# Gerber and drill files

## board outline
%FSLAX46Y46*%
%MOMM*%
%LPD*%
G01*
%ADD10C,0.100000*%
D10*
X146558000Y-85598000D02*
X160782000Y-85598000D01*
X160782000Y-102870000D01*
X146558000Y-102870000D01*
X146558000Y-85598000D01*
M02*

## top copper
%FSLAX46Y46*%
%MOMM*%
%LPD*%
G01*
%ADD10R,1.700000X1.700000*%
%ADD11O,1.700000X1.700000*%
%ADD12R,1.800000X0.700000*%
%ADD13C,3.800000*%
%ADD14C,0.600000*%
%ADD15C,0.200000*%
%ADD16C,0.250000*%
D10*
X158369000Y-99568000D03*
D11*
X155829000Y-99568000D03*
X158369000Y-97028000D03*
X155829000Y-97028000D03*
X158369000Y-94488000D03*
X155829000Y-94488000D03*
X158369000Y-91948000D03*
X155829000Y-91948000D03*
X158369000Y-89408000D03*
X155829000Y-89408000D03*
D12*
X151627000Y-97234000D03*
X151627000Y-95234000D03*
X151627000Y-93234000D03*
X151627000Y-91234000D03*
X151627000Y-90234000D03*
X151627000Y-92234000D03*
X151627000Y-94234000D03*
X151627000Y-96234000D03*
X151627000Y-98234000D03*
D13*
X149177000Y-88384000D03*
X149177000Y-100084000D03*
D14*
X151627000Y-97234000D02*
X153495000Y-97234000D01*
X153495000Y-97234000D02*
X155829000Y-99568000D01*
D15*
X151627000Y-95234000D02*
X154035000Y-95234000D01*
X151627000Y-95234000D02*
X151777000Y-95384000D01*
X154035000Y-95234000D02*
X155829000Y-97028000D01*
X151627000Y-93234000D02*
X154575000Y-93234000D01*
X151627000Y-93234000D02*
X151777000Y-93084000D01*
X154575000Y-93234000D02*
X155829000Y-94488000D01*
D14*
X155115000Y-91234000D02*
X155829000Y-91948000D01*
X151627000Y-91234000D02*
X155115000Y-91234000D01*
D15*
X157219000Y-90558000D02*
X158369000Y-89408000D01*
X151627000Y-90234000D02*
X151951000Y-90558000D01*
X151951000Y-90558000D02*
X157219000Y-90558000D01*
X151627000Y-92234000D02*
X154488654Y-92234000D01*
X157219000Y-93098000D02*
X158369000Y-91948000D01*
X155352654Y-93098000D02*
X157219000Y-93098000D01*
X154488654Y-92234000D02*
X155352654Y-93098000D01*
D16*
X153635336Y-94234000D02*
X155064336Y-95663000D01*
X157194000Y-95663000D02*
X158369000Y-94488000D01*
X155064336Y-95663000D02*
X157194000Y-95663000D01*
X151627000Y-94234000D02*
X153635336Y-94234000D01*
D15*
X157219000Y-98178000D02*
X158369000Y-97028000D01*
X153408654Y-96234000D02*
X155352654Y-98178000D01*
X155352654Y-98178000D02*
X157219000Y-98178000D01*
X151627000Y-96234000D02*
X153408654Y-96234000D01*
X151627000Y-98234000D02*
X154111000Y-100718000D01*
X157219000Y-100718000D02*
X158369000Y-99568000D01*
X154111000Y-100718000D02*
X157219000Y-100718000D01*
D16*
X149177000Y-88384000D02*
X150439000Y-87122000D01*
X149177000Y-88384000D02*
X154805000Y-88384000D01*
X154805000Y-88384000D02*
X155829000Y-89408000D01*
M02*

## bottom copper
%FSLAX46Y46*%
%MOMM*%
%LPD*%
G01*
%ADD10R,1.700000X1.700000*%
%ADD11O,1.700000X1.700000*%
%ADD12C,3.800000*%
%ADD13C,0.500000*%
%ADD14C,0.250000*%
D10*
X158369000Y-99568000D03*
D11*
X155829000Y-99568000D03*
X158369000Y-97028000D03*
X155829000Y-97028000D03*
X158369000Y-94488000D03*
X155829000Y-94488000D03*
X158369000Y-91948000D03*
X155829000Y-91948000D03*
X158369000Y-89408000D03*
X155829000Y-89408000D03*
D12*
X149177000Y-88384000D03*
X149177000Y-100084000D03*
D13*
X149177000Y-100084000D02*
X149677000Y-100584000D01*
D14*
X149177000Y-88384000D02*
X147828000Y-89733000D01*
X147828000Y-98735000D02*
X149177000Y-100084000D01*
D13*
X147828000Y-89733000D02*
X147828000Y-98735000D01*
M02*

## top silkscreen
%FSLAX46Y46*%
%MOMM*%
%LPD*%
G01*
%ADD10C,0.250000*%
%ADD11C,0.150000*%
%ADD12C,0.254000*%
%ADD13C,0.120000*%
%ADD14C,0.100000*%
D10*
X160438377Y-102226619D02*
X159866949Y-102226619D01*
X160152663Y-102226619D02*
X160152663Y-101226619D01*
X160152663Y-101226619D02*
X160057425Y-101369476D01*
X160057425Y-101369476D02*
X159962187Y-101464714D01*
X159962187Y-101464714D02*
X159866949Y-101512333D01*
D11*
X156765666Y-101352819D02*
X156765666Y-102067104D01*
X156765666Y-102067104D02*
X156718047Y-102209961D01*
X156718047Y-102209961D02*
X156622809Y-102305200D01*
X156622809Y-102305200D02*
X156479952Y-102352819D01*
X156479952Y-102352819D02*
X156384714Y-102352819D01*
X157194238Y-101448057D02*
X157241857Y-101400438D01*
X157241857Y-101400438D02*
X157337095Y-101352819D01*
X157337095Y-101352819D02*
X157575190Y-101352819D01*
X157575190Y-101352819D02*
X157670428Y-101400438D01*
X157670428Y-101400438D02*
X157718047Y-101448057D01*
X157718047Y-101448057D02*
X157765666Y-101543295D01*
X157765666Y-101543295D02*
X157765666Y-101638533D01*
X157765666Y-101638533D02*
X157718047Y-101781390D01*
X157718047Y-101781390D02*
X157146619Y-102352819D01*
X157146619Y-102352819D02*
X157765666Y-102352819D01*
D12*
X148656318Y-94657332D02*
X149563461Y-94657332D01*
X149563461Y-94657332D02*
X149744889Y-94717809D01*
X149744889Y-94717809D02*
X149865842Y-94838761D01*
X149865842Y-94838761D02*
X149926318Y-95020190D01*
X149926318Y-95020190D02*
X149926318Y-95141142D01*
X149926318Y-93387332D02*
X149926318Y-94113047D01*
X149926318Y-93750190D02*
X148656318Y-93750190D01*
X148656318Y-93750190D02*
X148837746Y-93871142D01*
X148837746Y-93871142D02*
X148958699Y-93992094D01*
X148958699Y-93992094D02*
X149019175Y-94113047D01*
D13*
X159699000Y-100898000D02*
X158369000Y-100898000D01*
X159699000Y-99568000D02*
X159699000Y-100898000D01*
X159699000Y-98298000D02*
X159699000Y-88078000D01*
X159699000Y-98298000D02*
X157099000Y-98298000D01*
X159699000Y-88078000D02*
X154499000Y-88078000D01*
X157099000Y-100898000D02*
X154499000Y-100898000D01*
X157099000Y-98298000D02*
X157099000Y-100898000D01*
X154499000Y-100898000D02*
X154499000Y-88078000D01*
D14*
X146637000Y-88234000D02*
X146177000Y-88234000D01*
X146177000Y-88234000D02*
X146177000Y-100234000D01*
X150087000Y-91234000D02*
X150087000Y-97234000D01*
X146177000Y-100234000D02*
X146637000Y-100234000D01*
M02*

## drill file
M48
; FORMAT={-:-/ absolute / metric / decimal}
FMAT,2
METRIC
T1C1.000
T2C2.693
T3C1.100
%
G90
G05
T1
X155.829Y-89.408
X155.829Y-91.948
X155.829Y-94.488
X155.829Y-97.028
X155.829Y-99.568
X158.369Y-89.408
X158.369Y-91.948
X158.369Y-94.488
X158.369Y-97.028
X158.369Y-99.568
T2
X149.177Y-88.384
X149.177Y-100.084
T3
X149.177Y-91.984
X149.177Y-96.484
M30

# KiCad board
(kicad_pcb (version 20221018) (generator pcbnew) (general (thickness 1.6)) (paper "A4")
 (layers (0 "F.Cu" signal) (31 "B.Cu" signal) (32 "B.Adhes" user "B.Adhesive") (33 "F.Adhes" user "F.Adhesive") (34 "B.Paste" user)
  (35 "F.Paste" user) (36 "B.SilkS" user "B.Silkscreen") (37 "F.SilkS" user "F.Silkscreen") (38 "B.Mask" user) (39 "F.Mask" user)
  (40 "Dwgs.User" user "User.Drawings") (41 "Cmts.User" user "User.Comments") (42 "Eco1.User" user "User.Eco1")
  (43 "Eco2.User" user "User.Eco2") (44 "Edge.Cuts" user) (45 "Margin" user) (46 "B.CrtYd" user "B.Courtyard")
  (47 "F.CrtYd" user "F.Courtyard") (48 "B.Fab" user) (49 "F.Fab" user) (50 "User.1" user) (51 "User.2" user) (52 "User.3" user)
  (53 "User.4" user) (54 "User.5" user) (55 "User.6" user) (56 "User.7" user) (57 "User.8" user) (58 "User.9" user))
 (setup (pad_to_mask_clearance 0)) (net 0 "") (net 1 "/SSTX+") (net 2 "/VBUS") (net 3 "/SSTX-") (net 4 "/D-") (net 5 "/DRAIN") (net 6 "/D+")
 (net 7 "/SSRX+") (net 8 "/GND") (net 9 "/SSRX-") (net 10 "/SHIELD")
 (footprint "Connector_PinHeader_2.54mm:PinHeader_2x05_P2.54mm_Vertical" (layer "F.Cu") (at 158.369 99.568 180)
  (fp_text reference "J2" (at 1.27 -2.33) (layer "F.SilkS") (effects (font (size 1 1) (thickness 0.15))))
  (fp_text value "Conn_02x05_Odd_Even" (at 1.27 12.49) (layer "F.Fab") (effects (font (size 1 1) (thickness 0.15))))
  (fp_line (start -1.33 -1.33) (end 0 -1.33) (stroke (width 0.12) (type solid)) (layer "F.SilkS"))
  (fp_line (start -1.33 0) (end -1.33 -1.33) (stroke (width 0.12) (type solid)) (layer "F.SilkS"))
  (fp_line (start -1.33 1.27) (end -1.33 11.49) (stroke (width 0.12) (type solid)) (layer "F.SilkS"))
  (fp_line (start -1.33 1.27) (end 1.27 1.27) (stroke (width 0.12) (type solid)) (layer "F.SilkS"))
  (fp_line (start -1.33 11.49) (end 3.87 11.49) (stroke (width 0.12) (type solid)) (layer "F.SilkS"))
  (fp_line (start 1.27 -1.33) (end 3.87 -1.33) (stroke (width 0.12) (type solid)) (layer "F.SilkS"))
  (fp_line (start 1.27 1.27) (end 1.27 -1.33) (stroke (width 0.12) (type solid)) (layer "F.SilkS"))
  (fp_line (start 3.87 -1.33) (end 3.87 11.49) (stroke (width 0.12) (type solid)) (layer "F.SilkS"))
  (pad "1" thru_hole rect (at 0 0 180) (size 1.7 1.7) (drill 1) (layers "*.Cu" "*.Mask") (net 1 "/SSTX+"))
  (pad "2" thru_hole oval (at 2.54 0 180) (size 1.7 1.7) (drill 1) (layers "*.Cu" "*.Mask") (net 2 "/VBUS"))
  (pad "3" thru_hole oval (at 0 2.54 180) (size 1.7 1.7) (drill 1) (layers "*.Cu" "*.Mask") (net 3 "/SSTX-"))
  (pad "4" thru_hole oval (at 2.54 2.54 180) (size 1.7 1.7) (drill 1) (layers "*.Cu" "*.Mask") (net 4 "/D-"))
  (pad "5" thru_hole oval (at 0 5.08 180) (size 1.7 1.7) (drill 1) (layers "*.Cu" "*.Mask") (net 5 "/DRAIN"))
  (pad "6" thru_hole oval (at 2.54 5.08 180) (size 1.7 1.7) (drill 1) (layers "*.Cu" "*.Mask") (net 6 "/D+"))
  (pad "7" thru_hole oval (at 0 7.62 180) (size 1.7 1.7) (drill 1) (layers "*.Cu" "*.Mask") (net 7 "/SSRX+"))
  (pad "8" thru_hole oval (at 2.54 7.62 180) (size 1.7 1.7) (drill 1) (layers "*.Cu" "*.Mask") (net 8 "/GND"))
  (pad "9" thru_hole oval (at 0 10.16 180) (size 1.7 1.7) (drill 1) (layers "*.Cu" "*.Mask") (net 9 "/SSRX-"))
  (pad "10" thru_hole oval (at 2.54 10.16 180) (size 1.7 1.7) (drill 1) (layers "*.Cu" "*.Mask") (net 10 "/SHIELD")))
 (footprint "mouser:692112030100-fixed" (layer "F.Cu") (at 149.352 94.234 -90)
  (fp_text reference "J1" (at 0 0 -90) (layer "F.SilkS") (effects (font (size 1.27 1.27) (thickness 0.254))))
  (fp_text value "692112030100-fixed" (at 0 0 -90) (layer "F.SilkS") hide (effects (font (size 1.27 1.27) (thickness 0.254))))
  (fp_line (start -6 2.715) (end -6 3.175) (stroke (width 0.1) (type solid)) (layer "F.SilkS"))
  (fp_line (start -6 3.175) (end 6 3.175) (stroke (width 0.1) (type solid)) (layer "F.SilkS"))
  (fp_line (start -3 -0.735) (end 3 -0.735) (stroke (width 0.1) (type solid)) (layer "F.SilkS"))
  (fp_line (start 6 3.175) (end 6 2.715) (stroke (width 0.1) (type solid)) (layer "F.SilkS"))
  (pad "" np_thru_hole circle (at -2.25 0.175 270) (size 0.001 0.001) (drill 1.1) (layers "*.Cu" "*.Mask"))
  (pad "" np_thru_hole circle (at 2.25 0.175 270) (size 0.001 0.001) (drill 1.1) (layers "*.Cu" "*.Mask"))
  (pad "1" smd rect (at 3 -2.275 270) (size 0.7 1.8) (layers "F.Cu" "F.Paste" "F.Mask") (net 2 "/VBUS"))
  (pad "2" smd rect (at 1 -2.275 270) (size 0.7 1.8) (layers "F.Cu" "F.Paste" "F.Mask") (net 4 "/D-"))
  (pad "3" smd rect (at -1 -2.275 270) (size 0.7 1.8) (layers "F.Cu" "F.Paste" "F.Mask") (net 6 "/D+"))
  (pad "4" smd rect (at -3 -2.275 270) (size 0.7 1.8) (layers "F.Cu" "F.Paste" "F.Mask") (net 8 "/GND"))
  (pad "5" smd rect (at -4 -2.275 270) (size 0.7 1.8) (layers "F.Cu" "F.Paste" "F.Mask") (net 9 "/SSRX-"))
  (pad "6" smd rect (at -2 -2.275 270) (size 0.7 1.8) (layers "F.Cu" "F.Paste" "F.Mask") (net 7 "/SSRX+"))
  (pad "7" smd rect (at 0 -2.275 270) (size 0.7 1.8) (layers "F.Cu" "F.Paste" "F.Mask") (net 5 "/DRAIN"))
  (pad "8" smd rect (at 2 -2.275 270) (size 0.7 1.8) (layers "F.Cu" "F.Paste" "F.Mask") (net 3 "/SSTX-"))
  (pad "9" smd rect (at 4 -2.275 270) (size 0.7 1.8) (layers "F.Cu" "F.Paste" "F.Mask") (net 1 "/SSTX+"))
  (pad "10" thru_hole circle (at -5.85 0.175 270) (size 3.8 3.8) (drill 2.6926) (layers "*.Cu" "*.Mask") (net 10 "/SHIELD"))
  (pad "11" thru_hole circle (at 5.85 0.175 270) (size 3.8 3.8) (drill 2.6926) (layers "*.Cu" "*.Mask") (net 10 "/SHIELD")))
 (gr_rect (start 146.558 85.598) (end 160.782 102.87) (stroke (width 0.1) (type solid)) (fill none) (layer "Edge.Cuts"))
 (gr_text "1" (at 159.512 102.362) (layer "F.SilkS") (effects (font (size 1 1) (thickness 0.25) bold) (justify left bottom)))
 (segment (start 151.627 97.234) (end 153.495 97.234) (width 0.6) (layer "F.Cu") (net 2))
 (segment (start 153.495 97.234) (end 155.829 99.568) (width 0.6) (layer "F.Cu") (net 2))
 (segment (start 151.627 95.234) (end 154.035 95.234) (width 0.2) (layer "F.Cu") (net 4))
 (segment (start 151.627 95.234) (end 151.777 95.384) (width 0.2) (layer "F.Cu") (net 4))
 (segment (start 154.035 95.234) (end 155.829 97.028) (width 0.2) (layer "F.Cu") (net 4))
 (segment (start 151.627 93.234) (end 154.575 93.234) (width 0.2) (layer "F.Cu") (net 6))
 (segment (start 151.627 93.234) (end 151.777 93.084) (width 0.2) (layer "F.Cu") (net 6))
 (segment (start 154.575 93.234) (end 155.829 94.488) (width 0.2) (layer "F.Cu") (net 6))
 (segment (start 155.115 91.234) (end 155.829 91.948) (width 0.6) (layer "F.Cu") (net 8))
 (segment (start 151.627 91.234) (end 155.115 91.234) (width 0.6) (layer "F.Cu") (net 8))
 (segment (start 157.219 90.558) (end 158.369 89.408) (width 0.2) (layer "F.Cu") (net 9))
 (segment (start 151.627 90.234) (end 151.951 90.558) (width 0.2) (layer "F.Cu") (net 9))
 (segment (start 151.951 90.558) (end 157.219 90.558) (width 0.2) (layer "F.Cu") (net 9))
 (segment (start 151.627 92.234) (end 154.488654 92.234) (width 0.2) (layer "F.Cu") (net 7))
 (segment (start 157.219 93.098) (end 158.369 91.948) (width 0.2) (layer "F.Cu") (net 7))
 (segment (start 155.352654 93.098) (end 157.219 93.098) (width 0.2) (layer "F.Cu") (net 7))
 (segment (start 154.488654 92.234) (end 155.352654 93.098) (width 0.2) (layer "F.Cu") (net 7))
 (segment (start 153.635336 94.234) (end 155.064336 95.663) (width 0.25) (layer "F.Cu") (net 5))
 (segment (start 157.194 95.663) (end 158.369 94.488) (width 0.25) (layer "F.Cu") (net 5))
 (segment (start 155.064336 95.663) (end 157.194 95.663) (width 0.25) (layer "F.Cu") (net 5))
 (segment (start 151.627 94.234) (end 153.635336 94.234) (width 0.25) (layer "F.Cu") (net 5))
 (segment (start 157.219 98.178) (end 158.369 97.028) (width 0.2) (layer "F.Cu") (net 3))
 (segment (start 153.408654 96.234) (end 155.352654 98.178) (width 0.2) (layer "F.Cu") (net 3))
 (segment (start 155.352654 98.178) (end 157.219 98.178) (width 0.2) (layer "F.Cu") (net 3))
 (segment (start 151.627 96.234) (end 153.408654 96.234) (width 0.2) (layer "F.Cu") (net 3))
 (segment (start 151.627 98.234) (end 154.111 100.718) (width 0.2) (layer "F.Cu") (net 1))
 (segment (start 157.219 100.718) (end 158.369 99.568) (width 0.2) (layer "F.Cu") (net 1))
 (segment (start 154.111 100.718) (end 157.219 100.718) (width 0.2) (layer "F.Cu") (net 1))
 (segment (start 149.177 88.384) (end 150.439 87.122) (width 0.25) (layer "F.Cu") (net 10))
 (segment (start 149.177 88.384) (end 154.805 88.384) (width 0.25) (layer "F.Cu") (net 10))
 (segment (start 154.805 88.384) (end 155.829 89.408) (width 0.25) (layer "F.Cu") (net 10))
 (segment (start 149.177 100.084) (end 149.677 100.584) (width 0.5) (layer "B.Cu") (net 10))
 (segment (start 149.177 88.384) (end 147.828 89.733) (width 0.25) (layer "B.Cu") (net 10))
 (segment (start 147.828 98.735) (end 149.177 100.084) (width 0.25) (layer "B.Cu") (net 10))
 (segment (start 147.828 89.733) (end 147.828 98.735) (width 0.5) (layer "B.Cu") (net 10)))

